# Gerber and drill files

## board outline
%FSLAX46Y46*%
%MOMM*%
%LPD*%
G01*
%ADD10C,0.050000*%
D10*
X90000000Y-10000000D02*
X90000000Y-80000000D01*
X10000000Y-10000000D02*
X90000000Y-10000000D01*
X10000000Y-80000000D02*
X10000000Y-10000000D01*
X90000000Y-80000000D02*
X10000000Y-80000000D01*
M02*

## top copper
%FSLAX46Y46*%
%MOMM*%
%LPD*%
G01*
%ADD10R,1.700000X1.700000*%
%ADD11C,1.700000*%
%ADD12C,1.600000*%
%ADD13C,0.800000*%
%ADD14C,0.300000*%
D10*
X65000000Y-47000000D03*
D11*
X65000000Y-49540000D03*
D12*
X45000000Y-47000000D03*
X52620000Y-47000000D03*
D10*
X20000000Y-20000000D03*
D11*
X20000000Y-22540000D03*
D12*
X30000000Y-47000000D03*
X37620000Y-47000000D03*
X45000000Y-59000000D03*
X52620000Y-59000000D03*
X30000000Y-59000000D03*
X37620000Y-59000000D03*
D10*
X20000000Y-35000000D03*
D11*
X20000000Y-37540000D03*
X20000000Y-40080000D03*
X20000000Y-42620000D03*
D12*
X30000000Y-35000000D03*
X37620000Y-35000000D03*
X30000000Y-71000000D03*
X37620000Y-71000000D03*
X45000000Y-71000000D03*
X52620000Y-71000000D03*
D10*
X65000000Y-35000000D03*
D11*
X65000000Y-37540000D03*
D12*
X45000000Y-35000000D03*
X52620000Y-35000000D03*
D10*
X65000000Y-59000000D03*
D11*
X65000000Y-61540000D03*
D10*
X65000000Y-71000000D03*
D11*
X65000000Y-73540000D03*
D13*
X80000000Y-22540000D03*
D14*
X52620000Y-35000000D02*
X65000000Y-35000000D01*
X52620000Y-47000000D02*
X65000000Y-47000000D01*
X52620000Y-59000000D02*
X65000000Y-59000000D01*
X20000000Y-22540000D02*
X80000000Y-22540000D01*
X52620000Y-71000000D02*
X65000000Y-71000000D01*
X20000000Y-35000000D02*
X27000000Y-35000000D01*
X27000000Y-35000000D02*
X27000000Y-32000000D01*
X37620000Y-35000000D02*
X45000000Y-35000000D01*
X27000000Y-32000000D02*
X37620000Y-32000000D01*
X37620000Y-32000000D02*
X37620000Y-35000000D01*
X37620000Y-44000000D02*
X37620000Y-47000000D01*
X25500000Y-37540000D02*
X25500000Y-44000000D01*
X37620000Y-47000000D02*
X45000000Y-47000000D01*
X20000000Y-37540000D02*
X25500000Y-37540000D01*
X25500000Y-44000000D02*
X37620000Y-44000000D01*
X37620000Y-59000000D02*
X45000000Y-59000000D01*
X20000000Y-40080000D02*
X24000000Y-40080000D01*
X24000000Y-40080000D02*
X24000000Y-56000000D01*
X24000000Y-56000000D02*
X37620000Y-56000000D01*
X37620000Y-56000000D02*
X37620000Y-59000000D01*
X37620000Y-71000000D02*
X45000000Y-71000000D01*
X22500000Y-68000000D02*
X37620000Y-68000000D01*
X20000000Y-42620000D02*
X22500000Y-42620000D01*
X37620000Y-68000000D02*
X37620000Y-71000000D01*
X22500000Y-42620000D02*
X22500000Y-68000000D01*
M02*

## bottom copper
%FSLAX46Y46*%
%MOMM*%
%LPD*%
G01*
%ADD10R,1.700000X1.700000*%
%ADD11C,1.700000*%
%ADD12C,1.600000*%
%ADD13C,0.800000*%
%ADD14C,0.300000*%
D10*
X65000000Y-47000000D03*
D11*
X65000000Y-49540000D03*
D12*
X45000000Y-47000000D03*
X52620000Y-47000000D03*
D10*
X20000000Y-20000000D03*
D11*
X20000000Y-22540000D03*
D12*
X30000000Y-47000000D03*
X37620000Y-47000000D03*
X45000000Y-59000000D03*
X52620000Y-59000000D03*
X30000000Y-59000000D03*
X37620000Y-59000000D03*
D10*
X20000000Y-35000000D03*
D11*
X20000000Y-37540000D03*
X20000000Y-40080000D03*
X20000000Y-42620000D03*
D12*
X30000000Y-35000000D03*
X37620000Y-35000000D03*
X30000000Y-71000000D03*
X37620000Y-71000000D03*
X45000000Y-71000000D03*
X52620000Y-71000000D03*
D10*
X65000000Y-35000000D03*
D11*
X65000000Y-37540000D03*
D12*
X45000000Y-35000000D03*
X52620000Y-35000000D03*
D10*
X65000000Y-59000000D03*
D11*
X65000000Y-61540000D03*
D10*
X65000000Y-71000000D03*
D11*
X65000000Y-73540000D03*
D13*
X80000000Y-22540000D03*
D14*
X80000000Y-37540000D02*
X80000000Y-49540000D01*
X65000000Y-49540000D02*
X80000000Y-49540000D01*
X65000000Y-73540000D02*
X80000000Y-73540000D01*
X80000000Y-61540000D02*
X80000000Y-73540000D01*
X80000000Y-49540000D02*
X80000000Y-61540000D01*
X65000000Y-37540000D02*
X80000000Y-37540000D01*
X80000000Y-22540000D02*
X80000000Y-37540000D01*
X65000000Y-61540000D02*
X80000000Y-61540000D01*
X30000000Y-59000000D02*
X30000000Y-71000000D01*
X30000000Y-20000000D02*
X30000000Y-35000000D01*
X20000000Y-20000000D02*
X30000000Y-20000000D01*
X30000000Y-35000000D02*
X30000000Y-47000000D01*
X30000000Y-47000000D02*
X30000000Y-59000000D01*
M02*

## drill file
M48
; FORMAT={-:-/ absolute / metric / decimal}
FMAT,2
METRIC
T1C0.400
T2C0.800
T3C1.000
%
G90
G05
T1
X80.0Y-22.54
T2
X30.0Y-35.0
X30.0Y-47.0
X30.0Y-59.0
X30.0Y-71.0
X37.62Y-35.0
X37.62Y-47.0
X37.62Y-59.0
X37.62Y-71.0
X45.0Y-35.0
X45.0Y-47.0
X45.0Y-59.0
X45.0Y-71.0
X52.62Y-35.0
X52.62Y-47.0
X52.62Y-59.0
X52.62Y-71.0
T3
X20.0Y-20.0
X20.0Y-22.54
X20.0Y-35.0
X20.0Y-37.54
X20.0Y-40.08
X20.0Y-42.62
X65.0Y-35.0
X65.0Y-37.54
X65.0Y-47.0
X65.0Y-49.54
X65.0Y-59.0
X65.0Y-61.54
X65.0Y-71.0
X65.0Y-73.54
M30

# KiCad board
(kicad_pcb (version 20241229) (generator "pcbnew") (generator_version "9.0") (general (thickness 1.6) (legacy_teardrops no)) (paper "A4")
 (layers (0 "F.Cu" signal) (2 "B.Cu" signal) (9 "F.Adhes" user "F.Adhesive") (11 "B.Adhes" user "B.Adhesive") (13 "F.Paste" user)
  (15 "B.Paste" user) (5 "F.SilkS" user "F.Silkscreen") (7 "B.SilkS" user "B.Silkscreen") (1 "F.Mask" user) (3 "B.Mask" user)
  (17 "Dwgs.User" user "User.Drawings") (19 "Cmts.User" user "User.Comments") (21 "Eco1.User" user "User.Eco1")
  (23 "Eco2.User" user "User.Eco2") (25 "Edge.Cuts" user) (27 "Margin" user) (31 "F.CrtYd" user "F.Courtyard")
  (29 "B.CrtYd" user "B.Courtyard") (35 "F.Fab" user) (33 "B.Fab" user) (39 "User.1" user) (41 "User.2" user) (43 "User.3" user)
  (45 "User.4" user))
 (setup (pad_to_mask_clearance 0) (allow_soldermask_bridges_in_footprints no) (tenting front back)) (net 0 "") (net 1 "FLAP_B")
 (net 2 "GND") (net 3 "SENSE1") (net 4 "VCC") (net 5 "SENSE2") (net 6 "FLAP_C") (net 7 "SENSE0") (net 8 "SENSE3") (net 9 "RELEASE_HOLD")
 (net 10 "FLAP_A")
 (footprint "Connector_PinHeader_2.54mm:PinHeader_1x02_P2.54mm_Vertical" (layer "F.Cu") (at 65 47)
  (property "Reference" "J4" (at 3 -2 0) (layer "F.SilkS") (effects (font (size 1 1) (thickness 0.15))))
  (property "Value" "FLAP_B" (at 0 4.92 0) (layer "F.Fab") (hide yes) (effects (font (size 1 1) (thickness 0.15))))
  (pad "1" thru_hole rect (at 0 0) (size 1.7 1.7) (drill 1) (layers "*.Cu" "*.Mask") (remove_unused_layers no) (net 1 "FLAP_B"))
  (pad "2" thru_hole circle (at 0 2.54) (size 1.7 1.7) (drill 1) (layers "*.Cu" "*.Mask") (remove_unused_layers no) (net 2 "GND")))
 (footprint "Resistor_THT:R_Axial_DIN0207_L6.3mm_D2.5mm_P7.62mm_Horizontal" (layer "F.Cu") (at 45 47)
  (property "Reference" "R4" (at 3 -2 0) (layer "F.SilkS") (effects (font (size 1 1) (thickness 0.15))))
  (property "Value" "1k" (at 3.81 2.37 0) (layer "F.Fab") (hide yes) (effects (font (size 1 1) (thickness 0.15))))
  (pad "1" thru_hole circle (at 0 0) (size 1.6 1.6) (drill 0.8) (layers "*.Cu" "*.Mask") (remove_unused_layers no) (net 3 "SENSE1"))
  (pad "2" thru_hole circle (at 7.62 0) (size 1.6 1.6) (drill 0.8) (layers "*.Cu" "*.Mask") (remove_unused_layers no) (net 1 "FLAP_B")))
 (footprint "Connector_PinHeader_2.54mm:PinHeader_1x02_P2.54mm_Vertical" (layer "F.Cu") (at 20 20)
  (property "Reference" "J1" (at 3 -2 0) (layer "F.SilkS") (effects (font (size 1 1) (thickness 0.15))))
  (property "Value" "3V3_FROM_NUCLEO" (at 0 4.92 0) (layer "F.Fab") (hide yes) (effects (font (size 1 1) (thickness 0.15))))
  (pad "1" thru_hole rect (at 0 0) (size 1.7 1.7) (drill 1) (layers "*.Cu" "*.Mask") (remove_unused_layers no) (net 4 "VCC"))
  (pad "2" thru_hole circle (at 0 2.54) (size 1.7 1.7) (drill 1) (layers "*.Cu" "*.Mask") (remove_unused_layers no) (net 2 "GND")))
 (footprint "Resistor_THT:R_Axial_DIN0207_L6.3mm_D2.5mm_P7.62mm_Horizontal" (layer "F.Cu") (at 30 47)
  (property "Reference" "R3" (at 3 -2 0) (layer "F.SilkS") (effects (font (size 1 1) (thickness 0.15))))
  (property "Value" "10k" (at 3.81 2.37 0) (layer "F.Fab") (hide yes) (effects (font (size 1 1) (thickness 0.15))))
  (pad "1" thru_hole circle (at 0 0) (size 1.6 1.6) (drill 0.8) (layers "*.Cu" "*.Mask") (remove_unused_layers no) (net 4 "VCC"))
  (pad "2" thru_hole circle (at 7.62 0) (size 1.6 1.6) (drill 0.8) (layers "*.Cu" "*.Mask") (remove_unused_layers no) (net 3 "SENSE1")))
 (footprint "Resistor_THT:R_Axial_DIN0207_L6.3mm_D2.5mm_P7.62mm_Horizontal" (layer "F.Cu") (at 45 59)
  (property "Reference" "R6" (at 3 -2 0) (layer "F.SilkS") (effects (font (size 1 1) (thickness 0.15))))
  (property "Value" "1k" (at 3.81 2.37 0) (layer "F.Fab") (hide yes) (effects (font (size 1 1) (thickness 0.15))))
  (pad "1" thru_hole circle (at 0 0) (size 1.6 1.6) (drill 0.8) (layers "*.Cu" "*.Mask") (remove_unused_layers no) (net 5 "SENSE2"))
  (pad "2" thru_hole circle (at 7.62 0) (size 1.6 1.6) (drill 0.8) (layers "*.Cu" "*.Mask") (remove_unused_layers no) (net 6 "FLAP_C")))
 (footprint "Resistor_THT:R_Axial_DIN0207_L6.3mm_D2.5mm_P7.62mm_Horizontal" (layer "F.Cu") (at 30 59)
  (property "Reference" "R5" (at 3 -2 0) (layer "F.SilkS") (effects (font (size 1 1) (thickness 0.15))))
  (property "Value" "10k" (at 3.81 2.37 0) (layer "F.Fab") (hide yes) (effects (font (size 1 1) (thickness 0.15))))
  (pad "1" thru_hole circle (at 0 0) (size 1.6 1.6) (drill 0.8) (layers "*.Cu" "*.Mask") (remove_unused_layers no) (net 4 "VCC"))
  (pad "2" thru_hole circle (at 7.62 0) (size 1.6 1.6) (drill 0.8) (layers "*.Cu" "*.Mask") (remove_unused_layers no) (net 5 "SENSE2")))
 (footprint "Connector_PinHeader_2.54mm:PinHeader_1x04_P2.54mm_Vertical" (layer "F.Cu") (at 20 35)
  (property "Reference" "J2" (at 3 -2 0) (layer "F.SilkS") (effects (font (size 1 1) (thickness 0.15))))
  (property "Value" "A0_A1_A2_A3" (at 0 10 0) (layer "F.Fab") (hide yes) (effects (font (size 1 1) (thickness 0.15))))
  (pad "1" thru_hole rect (at 0 0) (size 1.7 1.7) (drill 1) (layers "*.Cu" "*.Mask") (remove_unused_layers no) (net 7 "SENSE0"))
  (pad "2" thru_hole circle (at 0 2.54) (size 1.7 1.7) (drill 1) (layers "*.Cu" "*.Mask") (remove_unused_layers no) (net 3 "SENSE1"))
  (pad "3" thru_hole circle (at 0 5.08) (size 1.7 1.7) (drill 1) (layers "*.Cu" "*.Mask") (remove_unused_layers no) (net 5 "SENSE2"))
  (pad "4" thru_hole circle (at 0 7.62) (size 1.7 1.7) (drill 1) (layers "*.Cu" "*.Mask") (remove_unused_layers no) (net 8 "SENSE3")))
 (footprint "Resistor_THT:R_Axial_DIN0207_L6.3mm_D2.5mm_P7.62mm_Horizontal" (layer "F.Cu") (at 30 35)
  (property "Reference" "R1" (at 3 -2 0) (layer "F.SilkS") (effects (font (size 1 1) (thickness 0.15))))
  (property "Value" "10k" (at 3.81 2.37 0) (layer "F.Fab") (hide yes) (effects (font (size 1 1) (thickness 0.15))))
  (pad "1" thru_hole circle (at 0 0) (size 1.6 1.6) (drill 0.8) (layers "*.Cu" "*.Mask") (remove_unused_layers no) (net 4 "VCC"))
  (pad "2" thru_hole circle (at 7.62 0) (size 1.6 1.6) (drill 0.8) (layers "*.Cu" "*.Mask") (remove_unused_layers no) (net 7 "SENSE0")))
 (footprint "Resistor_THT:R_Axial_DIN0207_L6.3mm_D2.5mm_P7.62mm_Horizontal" (layer "F.Cu") (at 30 71)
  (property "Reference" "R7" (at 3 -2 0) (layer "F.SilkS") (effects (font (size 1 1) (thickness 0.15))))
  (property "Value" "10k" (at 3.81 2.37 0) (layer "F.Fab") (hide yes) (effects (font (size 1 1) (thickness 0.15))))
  (pad "1" thru_hole circle (at 0 0) (size 1.6 1.6) (drill 0.8) (layers "*.Cu" "*.Mask") (remove_unused_layers no) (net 4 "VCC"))
  (pad "2" thru_hole circle (at 7.62 0) (size 1.6 1.6) (drill 0.8) (layers "*.Cu" "*.Mask") (remove_unused_layers no) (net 8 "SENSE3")))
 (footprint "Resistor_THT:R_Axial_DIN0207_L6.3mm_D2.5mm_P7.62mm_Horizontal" (layer "F.Cu") (at 45 71)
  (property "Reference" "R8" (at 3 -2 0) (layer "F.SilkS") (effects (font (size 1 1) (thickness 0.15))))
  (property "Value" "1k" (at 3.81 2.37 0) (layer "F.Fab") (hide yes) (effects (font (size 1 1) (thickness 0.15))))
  (pad "1" thru_hole circle (at 0 0) (size 1.6 1.6) (drill 0.8) (layers "*.Cu" "*.Mask") (remove_unused_layers no) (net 8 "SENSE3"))
  (pad "2" thru_hole circle (at 7.62 0) (size 1.6 1.6) (drill 0.8) (layers "*.Cu" "*.Mask") (remove_unused_layers no) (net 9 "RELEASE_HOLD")))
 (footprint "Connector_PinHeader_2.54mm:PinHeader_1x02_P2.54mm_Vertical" (layer "F.Cu") (at 65 35)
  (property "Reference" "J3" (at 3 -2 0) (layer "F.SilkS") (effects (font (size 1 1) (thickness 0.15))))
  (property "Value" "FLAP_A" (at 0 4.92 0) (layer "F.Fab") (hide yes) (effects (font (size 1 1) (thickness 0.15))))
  (pad "1" thru_hole rect (at 0 0) (size 1.7 1.7) (drill 1) (layers "*.Cu" "*.Mask") (remove_unused_layers no) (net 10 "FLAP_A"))
  (pad "2" thru_hole circle (at 0 2.54) (size 1.7 1.7) (drill 1) (layers "*.Cu" "*.Mask") (remove_unused_layers no) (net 2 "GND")))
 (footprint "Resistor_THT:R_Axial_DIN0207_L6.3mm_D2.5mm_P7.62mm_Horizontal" (layer "F.Cu") (at 45 35)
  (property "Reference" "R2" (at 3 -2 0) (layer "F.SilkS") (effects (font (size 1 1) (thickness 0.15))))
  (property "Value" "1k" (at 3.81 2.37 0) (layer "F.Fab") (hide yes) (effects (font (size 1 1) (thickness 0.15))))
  (pad "1" thru_hole circle (at 0 0) (size 1.6 1.6) (drill 0.8) (layers "*.Cu" "*.Mask") (remove_unused_layers no) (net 7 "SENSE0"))
  (pad "2" thru_hole circle (at 7.62 0) (size 1.6 1.6) (drill 0.8) (layers "*.Cu" "*.Mask") (remove_unused_layers no) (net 10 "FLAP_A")))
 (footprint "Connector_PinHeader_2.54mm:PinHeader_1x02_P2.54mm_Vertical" (layer "F.Cu") (at 65 59)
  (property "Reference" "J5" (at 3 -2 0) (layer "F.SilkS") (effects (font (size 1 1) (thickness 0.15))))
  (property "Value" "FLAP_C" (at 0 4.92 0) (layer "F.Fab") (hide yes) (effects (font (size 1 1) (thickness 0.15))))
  (pad "1" thru_hole rect (at 0 0) (size 1.7 1.7) (drill 1) (layers "*.Cu" "*.Mask") (remove_unused_layers no) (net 6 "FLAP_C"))
  (pad "2" thru_hole circle (at 0 2.54) (size 1.7 1.7) (drill 1) (layers "*.Cu" "*.Mask") (remove_unused_layers no) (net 2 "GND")))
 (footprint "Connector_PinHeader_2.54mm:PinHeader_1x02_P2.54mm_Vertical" (layer "F.Cu") (at 65 71)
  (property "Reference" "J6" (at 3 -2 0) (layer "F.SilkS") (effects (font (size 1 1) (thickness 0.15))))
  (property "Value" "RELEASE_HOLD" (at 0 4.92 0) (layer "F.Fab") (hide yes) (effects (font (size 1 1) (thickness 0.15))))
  (pad "1" thru_hole rect (at 0 0) (size 1.7 1.7) (drill 1) (layers "*.Cu" "*.Mask") (remove_unused_layers no) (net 9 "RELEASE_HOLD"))
  (pad "2" thru_hole circle (at 0 2.54) (size 1.7 1.7) (drill 1) (layers "*.Cu" "*.Mask") (remove_unused_layers no) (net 2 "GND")))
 (gr_line (start 90 10) (end 90 80) (stroke (width 0.05) (type default)) (layer "Edge.Cuts"))
 (gr_line (start 10 10) (end 90 10) (stroke (width 0.05) (type default)) (layer "Edge.Cuts"))
 (gr_line (start 10 80) (end 10 10) (stroke (width 0.05) (type default)) (layer "Edge.Cuts"))
 (gr_line (start 90 80) (end 10 80) (stroke (width 0.05) (type default)) (layer "Edge.Cuts"))
 (segment (start 52.62 35) (end 65 35) (width 0.3) (layer "F.Cu") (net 10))
 (segment (start 52.62 47) (end 65 47) (width 0.3) (layer "F.Cu") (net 1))
 (segment (start 52.62 59) (end 65 59) (width 0.3) (layer "F.Cu") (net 6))
 (segment (start 20 22.54) (end 80 22.54) (width 0.3) (layer "F.Cu") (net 2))
 (via (at 80 22.54) (size 0.8) (drill 0.4) (layers "F.Cu" "B.Cu") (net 2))
 (segment (start 80 37.54) (end 80 49.54) (width 0.3) (layer "B.Cu") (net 2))
 (segment (start 65 49.54) (end 80 49.54) (width 0.3) (layer "B.Cu") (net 2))
 (segment (start 65 73.54) (end 80 73.54) (width 0.3) (layer "B.Cu") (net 2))
 (segment (start 80 61.54) (end 80 73.54) (width 0.3) (layer "B.Cu") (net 2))
 (segment (start 80 49.54) (end 80 61.54) (width 0.3) (layer "B.Cu") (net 2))
 (segment (start 65 37.54) (end 80 37.54) (width 0.3) (layer "B.Cu") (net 2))
 (segment (start 80 22.54) (end 80 37.54) (width 0.3) (layer "B.Cu") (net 2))
 (segment (start 65 61.54) (end 80 61.54) (width 0.3) (layer "B.Cu") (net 2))
 (segment (start 52.62 71) (end 65 71) (width 0.3) (layer "F.Cu") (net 9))
 (segment (start 20 35) (end 27 35) (width 0.3) (layer "F.Cu") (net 7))
 (segment (start 27 35) (end 27 32) (width 0.3) (layer "F.Cu") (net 7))
 (segment (start 37.62 35) (end 45 35) (width 0.3) (layer "F.Cu") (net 7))
 (segment (start 27 32) (end 37.62 32) (width 0.3) (layer "F.Cu") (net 7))
 (segment (start 37.62 32) (end 37.62 35) (width 0.3) (layer "F.Cu") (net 7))
 (segment (start 37.62 44) (end 37.62 47) (width 0.3) (layer "F.Cu") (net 3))
 (segment (start 25.5 37.54) (end 25.5 44) (width 0.3) (layer "F.Cu") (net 3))
 (segment (start 37.62 47) (end 45 47) (width 0.3) (layer "F.Cu") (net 3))
 (segment (start 20 37.54) (end 25.5 37.54) (width 0.3) (layer "F.Cu") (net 3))
 (segment (start 25.5 44) (end 37.62 44) (width 0.3) (layer "F.Cu") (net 3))
 (segment (start 37.62 59) (end 45 59) (width 0.3) (layer "F.Cu") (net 5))
 (segment (start 20 40.08) (end 24 40.08) (width 0.3) (layer "F.Cu") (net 5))
 (segment (start 24 40.08) (end 24 56) (width 0.3) (layer "F.Cu") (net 5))
 (segment (start 24 56) (end 37.62 56) (width 0.3) (layer "F.Cu") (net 5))
 (segment (start 37.62 56) (end 37.62 59) (width 0.3) (layer "F.Cu") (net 5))
 (segment (start 37.62 71) (end 45 71) (width 0.3) (layer "F.Cu") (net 8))
 (segment (start 22.5 68) (end 37.62 68) (width 0.3) (layer "F.Cu") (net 8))
 (segment (start 20 42.62) (end 22.5 42.62) (width 0.3) (layer "F.Cu") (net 8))
 (segment (start 37.62 68) (end 37.62 71) (width 0.3) (layer "F.Cu") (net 8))
 (segment (start 22.5 42.62) (end 22.5 68) (width 0.3) (layer "F.Cu") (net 8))
 (segment (start 30 59) (end 30 71) (width 0.3) (layer "B.Cu") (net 4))
 (segment (start 30 20) (end 30 35) (width 0.3) (layer "B.Cu") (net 4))
 (segment (start 20 20) (end 30 20) (width 0.3) (layer "B.Cu") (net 4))
 (segment (start 30 35) (end 30 47) (width 0.3) (layer "B.Cu") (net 4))
 (segment (start 30 47) (end 30 59) (width 0.3) (layer "B.Cu") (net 4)))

